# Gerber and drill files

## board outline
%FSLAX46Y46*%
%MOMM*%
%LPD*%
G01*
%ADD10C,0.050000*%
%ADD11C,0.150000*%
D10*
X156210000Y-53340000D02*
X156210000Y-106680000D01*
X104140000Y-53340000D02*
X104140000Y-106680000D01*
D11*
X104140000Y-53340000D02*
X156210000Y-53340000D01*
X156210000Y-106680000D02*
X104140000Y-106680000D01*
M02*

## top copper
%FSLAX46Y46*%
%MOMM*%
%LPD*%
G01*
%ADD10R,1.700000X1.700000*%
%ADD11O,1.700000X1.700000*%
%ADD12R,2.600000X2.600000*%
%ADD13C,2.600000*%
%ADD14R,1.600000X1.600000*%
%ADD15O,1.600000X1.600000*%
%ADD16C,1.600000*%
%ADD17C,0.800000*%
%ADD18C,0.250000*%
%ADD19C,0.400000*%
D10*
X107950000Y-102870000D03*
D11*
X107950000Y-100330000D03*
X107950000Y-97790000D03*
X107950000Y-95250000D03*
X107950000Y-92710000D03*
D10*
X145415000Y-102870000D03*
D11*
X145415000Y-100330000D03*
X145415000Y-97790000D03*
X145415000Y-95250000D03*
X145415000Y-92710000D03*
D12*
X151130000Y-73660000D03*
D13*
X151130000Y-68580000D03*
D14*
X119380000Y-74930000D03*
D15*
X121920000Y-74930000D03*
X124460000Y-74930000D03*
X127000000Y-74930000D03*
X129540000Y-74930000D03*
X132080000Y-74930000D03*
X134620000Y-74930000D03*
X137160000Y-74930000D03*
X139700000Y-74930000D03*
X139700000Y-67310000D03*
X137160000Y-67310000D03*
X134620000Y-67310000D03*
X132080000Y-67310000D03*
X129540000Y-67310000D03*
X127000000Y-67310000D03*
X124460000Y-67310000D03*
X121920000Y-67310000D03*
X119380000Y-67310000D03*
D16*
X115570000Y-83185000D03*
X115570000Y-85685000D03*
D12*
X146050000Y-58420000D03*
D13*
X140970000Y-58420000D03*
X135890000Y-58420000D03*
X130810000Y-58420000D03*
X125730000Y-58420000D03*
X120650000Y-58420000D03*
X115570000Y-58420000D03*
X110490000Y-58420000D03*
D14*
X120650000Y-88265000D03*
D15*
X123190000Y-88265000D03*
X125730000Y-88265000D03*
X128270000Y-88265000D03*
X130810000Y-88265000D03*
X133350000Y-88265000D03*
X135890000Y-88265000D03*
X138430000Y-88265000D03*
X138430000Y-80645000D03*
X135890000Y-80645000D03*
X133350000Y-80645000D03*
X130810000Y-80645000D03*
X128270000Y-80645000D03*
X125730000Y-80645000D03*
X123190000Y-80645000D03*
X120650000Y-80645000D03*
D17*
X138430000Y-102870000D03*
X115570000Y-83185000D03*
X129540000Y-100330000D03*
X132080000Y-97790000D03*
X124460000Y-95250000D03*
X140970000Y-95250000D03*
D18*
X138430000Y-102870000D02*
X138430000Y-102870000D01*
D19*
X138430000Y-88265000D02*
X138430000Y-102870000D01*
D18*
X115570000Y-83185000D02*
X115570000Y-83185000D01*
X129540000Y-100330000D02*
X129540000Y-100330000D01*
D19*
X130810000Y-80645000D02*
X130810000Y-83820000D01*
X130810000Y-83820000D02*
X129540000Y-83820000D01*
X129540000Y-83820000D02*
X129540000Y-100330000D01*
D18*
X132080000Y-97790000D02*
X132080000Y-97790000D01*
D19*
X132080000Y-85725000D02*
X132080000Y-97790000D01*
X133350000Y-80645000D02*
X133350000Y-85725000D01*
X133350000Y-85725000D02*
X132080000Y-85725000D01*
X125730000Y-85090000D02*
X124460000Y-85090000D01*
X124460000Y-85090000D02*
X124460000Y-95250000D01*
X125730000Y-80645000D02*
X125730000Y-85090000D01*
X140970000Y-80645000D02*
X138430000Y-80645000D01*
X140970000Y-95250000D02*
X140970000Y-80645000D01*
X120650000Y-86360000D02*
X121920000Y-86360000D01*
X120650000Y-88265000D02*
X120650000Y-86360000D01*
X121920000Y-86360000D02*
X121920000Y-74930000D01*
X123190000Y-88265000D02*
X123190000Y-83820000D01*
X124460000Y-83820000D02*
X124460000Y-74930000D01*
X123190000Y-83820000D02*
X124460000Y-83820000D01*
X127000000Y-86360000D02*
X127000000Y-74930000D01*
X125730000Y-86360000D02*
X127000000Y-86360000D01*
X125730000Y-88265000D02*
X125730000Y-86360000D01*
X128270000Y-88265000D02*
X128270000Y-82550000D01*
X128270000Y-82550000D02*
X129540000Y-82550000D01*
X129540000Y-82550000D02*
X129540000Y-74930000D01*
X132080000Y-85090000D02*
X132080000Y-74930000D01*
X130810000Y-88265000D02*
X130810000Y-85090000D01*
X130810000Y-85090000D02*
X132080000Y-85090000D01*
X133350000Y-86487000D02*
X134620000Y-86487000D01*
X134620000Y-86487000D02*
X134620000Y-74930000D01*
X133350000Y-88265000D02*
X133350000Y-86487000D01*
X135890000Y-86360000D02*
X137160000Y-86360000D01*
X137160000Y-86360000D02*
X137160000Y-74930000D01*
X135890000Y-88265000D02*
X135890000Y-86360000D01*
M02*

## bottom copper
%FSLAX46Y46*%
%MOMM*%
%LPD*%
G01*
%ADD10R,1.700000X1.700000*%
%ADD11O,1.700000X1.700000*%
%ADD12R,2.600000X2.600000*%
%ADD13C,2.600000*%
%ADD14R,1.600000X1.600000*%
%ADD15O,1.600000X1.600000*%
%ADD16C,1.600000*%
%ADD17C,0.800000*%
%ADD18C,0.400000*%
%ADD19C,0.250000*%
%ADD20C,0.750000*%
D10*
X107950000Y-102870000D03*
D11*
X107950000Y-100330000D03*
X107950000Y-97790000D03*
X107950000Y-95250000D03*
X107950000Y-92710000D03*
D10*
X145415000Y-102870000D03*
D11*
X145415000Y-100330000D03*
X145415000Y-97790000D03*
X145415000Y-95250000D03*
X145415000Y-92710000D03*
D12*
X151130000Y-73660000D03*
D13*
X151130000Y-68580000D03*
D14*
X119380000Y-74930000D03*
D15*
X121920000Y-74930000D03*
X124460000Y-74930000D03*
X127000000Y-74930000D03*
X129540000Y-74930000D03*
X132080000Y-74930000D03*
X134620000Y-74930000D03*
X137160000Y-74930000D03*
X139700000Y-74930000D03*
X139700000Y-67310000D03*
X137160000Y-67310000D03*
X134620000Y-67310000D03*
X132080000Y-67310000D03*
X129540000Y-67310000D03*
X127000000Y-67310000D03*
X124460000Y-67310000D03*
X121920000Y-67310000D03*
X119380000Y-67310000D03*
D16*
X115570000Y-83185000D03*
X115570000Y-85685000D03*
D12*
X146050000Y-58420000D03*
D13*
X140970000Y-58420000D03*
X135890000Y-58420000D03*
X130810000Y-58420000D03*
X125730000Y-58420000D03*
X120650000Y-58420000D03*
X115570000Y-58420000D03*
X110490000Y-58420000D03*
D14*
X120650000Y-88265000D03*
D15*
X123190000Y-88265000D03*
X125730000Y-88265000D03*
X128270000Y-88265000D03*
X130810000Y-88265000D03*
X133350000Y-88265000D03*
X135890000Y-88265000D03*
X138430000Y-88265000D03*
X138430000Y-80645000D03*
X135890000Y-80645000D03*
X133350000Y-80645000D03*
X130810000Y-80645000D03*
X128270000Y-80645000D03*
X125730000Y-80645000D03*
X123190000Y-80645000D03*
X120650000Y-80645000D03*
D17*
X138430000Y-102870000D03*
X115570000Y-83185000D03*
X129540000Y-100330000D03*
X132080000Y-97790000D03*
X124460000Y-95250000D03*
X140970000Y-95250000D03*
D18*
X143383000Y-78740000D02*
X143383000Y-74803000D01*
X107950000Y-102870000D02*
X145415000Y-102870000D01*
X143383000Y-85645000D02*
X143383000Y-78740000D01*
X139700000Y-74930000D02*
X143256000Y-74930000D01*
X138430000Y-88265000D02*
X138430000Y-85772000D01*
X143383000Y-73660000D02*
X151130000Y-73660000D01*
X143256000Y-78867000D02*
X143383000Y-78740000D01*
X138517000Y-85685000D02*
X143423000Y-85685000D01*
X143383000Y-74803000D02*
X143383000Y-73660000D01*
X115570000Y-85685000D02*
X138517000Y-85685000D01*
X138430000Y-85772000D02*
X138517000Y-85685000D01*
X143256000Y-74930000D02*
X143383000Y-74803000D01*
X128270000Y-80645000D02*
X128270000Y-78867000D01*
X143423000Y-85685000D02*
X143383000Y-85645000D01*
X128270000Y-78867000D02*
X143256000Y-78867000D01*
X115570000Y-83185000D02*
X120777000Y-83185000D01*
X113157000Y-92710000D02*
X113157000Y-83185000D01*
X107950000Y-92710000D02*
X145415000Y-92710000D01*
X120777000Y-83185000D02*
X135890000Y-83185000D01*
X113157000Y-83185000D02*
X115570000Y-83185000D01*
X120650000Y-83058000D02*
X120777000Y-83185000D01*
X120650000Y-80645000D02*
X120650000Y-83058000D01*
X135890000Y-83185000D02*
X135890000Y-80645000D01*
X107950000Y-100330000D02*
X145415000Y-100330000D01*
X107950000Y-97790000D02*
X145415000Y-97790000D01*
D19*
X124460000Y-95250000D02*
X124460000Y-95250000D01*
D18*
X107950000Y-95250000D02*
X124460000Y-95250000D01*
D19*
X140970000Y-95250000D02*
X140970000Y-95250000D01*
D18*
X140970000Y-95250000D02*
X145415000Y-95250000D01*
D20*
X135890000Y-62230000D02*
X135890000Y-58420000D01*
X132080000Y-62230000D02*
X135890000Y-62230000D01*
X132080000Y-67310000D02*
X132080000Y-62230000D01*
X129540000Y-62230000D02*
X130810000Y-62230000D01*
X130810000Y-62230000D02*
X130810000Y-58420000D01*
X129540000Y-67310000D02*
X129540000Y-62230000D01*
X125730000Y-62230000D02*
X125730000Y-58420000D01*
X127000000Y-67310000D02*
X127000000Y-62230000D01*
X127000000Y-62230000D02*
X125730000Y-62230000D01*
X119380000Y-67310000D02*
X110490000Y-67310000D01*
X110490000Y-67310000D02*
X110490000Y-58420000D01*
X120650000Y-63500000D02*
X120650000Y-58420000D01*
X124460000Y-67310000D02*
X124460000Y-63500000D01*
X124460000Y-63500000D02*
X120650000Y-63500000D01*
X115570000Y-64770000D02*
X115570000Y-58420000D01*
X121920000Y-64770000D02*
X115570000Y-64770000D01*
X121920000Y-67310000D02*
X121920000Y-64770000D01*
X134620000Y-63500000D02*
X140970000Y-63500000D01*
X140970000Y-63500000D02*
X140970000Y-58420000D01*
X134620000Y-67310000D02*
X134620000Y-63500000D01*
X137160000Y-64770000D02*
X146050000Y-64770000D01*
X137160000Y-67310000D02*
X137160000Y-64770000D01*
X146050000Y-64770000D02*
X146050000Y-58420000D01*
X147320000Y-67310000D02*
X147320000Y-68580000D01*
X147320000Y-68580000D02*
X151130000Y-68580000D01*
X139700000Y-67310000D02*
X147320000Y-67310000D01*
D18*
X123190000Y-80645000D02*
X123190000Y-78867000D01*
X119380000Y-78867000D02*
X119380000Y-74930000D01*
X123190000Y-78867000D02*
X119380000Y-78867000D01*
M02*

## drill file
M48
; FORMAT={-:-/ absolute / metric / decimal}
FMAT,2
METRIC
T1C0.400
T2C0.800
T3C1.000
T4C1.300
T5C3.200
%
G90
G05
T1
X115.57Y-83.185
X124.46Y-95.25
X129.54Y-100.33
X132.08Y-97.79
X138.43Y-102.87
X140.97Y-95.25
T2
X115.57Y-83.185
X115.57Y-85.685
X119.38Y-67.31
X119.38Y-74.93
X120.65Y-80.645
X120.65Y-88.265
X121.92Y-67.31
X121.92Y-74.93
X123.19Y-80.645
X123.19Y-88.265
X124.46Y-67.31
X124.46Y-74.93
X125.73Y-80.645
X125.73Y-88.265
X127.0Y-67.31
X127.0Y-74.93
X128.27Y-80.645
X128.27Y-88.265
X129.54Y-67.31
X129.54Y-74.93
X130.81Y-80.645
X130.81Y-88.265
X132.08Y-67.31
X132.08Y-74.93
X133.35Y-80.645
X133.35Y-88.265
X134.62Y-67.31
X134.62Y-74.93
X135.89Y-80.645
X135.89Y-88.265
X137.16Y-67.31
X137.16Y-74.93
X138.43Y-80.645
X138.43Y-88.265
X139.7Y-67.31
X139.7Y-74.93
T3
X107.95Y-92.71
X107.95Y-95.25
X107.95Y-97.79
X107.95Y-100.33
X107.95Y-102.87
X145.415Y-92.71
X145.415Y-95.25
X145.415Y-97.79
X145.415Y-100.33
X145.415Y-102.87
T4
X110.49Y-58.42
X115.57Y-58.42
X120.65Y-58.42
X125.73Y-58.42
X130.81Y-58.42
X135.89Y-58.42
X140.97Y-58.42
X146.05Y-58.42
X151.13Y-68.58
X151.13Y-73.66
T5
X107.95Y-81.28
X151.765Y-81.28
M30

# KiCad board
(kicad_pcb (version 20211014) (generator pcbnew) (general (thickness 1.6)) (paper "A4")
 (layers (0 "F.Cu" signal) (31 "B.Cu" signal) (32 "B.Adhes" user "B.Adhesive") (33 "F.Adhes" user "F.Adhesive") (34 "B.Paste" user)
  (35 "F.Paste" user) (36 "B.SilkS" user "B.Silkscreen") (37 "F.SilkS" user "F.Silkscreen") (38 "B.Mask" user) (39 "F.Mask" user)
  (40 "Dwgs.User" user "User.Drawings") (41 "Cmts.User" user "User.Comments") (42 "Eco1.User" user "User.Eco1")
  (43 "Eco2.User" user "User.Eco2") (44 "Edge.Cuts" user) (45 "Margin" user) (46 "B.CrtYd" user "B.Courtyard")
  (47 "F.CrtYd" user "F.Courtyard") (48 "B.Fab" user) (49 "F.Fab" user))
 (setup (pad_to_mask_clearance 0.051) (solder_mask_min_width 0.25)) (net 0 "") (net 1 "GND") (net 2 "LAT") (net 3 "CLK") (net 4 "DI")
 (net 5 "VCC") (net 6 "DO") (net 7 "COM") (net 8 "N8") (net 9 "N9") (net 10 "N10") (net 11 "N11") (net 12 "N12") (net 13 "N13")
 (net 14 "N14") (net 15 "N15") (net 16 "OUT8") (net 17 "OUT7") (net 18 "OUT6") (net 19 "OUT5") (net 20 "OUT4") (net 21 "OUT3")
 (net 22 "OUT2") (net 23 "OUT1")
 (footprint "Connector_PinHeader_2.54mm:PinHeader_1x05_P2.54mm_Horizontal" (layer "F.Cu") (at 107.95 102.87 180)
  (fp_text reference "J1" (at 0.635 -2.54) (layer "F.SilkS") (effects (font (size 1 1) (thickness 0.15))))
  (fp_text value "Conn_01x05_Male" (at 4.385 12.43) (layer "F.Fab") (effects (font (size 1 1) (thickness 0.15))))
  (pad "1" thru_hole rect locked (at 0 0 180) (size 1.7 1.7) (drill 1) (layers *.Cu *.Mask) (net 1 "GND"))
  (pad "2" thru_hole oval locked (at 0 2.54 180) (size 1.7 1.7) (drill 1) (layers *.Cu *.Mask) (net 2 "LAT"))
  (pad "3" thru_hole oval locked (at 0 5.08 180) (size 1.7 1.7) (drill 1) (layers *.Cu *.Mask) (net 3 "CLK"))
  (pad "4" thru_hole oval locked (at 0 7.62 180) (size 1.7 1.7) (drill 1) (layers *.Cu *.Mask) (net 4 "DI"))
  (pad "5" thru_hole oval locked (at 0 10.16 180) (size 1.7 1.7) (drill 1) (layers *.Cu *.Mask) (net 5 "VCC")))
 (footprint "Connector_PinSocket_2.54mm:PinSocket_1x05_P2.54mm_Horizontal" (layer "F.Cu") (at 145.415 102.87 180)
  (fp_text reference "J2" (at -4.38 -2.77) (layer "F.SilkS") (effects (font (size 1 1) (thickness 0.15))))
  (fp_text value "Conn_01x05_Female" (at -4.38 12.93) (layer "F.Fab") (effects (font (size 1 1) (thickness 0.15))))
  (pad "1" thru_hole rect locked (at 0 0 180) (size 1.7 1.7) (drill 1) (layers *.Cu *.Mask) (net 1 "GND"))
  (pad "2" thru_hole oval locked (at 0 2.54 180) (size 1.7 1.7) (drill 1) (layers *.Cu *.Mask) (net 2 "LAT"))
  (pad "3" thru_hole oval locked (at 0 5.08 180) (size 1.7 1.7) (drill 1) (layers *.Cu *.Mask) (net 3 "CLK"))
  (pad "4" thru_hole oval locked (at 0 7.62 180) (size 1.7 1.7) (drill 1) (layers *.Cu *.Mask) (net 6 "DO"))
  (pad "5" thru_hole oval locked (at 0 10.16 180) (size 1.7 1.7) (drill 1) (layers *.Cu *.Mask) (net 5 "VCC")))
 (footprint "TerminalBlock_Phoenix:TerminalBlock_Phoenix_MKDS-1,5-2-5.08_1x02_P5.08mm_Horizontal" (layer "F.Cu") (at 151.13 73.66 90)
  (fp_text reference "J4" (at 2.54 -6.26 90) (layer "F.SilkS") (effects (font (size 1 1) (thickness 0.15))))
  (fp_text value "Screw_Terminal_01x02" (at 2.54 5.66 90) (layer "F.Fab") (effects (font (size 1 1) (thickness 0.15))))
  (pad "1" thru_hole rect locked (at 0 0 90) (size 2.6 2.6) (drill 1.3) (layers *.Cu *.Mask) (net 1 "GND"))
  (pad "2" thru_hole circle locked (at 5.08 0 90) (size 2.6 2.6) (drill 1.3) (layers *.Cu *.Mask) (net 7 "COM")))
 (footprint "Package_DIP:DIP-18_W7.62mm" (layer "F.Cu") (at 119.38 74.93 90)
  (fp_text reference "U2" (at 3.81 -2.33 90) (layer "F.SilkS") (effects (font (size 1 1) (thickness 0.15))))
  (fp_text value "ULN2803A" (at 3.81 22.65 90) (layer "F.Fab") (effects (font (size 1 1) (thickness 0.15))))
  (pad "1" thru_hole rect locked (at 0 0 90) (size 1.6 1.6) (drill 0.8) (layers *.Cu *.Mask) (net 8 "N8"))
  (pad "2" thru_hole oval locked (at 0 2.54 90) (size 1.6 1.6) (drill 0.8) (layers *.Cu *.Mask) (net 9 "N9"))
  (pad "3" thru_hole oval locked (at 0 5.08 90) (size 1.6 1.6) (drill 0.8) (layers *.Cu *.Mask) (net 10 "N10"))
  (pad "4" thru_hole oval locked (at 0 7.62 90) (size 1.6 1.6) (drill 0.8) (layers *.Cu *.Mask) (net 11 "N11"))
  (pad "5" thru_hole oval locked (at 0 10.16 90) (size 1.6 1.6) (drill 0.8) (layers *.Cu *.Mask) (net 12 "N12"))
  (pad "6" thru_hole oval locked (at 0 12.7 90) (size 1.6 1.6) (drill 0.8) (layers *.Cu *.Mask) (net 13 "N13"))
  (pad "7" thru_hole oval locked (at 0 15.24 90) (size 1.6 1.6) (drill 0.8) (layers *.Cu *.Mask) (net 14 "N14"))
  (pad "8" thru_hole oval locked (at 0 17.78 90) (size 1.6 1.6) (drill 0.8) (layers *.Cu *.Mask) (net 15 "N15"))
  (pad "9" thru_hole oval locked (at 0 20.32 90) (size 1.6 1.6) (drill 0.8) (layers *.Cu *.Mask) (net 1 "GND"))
  (pad "10" thru_hole oval locked (at 7.62 20.32 90) (size 1.6 1.6) (drill 0.8) (layers *.Cu *.Mask) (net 7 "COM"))
  (pad "11" thru_hole oval locked (at 7.62 17.78 90) (size 1.6 1.6) (drill 0.8) (layers *.Cu *.Mask) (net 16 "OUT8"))
  (pad "12" thru_hole oval locked (at 7.62 15.24 90) (size 1.6 1.6) (drill 0.8) (layers *.Cu *.Mask) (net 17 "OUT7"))
  (pad "13" thru_hole oval locked (at 7.62 12.7 90) (size 1.6 1.6) (drill 0.8) (layers *.Cu *.Mask) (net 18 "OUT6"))
  (pad "14" thru_hole oval locked (at 7.62 10.16 90) (size 1.6 1.6) (drill 0.8) (layers *.Cu *.Mask) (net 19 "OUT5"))
  (pad "15" thru_hole oval locked (at 7.62 7.62 90) (size 1.6 1.6) (drill 0.8) (layers *.Cu *.Mask) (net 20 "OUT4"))
  (pad "16" thru_hole oval locked (at 7.62 5.08 90) (size 1.6 1.6) (drill 0.8) (layers *.Cu *.Mask) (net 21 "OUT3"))
  (pad "17" thru_hole oval locked (at 7.62 2.54 90) (size 1.6 1.6) (drill 0.8) (layers *.Cu *.Mask) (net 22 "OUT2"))
  (pad "18" thru_hole oval locked (at 7.62 0 90) (size 1.6 1.6) (drill 0.8) (layers *.Cu *.Mask) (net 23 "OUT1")))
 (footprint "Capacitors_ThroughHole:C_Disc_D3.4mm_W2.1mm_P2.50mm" (layer "F.Cu") (at 115.57 83.185 -90)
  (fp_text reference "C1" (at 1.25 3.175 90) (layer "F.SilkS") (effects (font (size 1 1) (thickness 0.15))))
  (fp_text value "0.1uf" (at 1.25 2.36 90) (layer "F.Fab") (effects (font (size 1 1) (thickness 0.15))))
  (pad "1" thru_hole circle locked (at 0 0 270) (size 1.6 1.6) (drill 0.8) (layers *.Cu *.Mask) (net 5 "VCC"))
  (pad "2" thru_hole circle locked (at 2.5 0 270) (size 1.6 1.6) (drill 0.8) (layers *.Cu *.Mask) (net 1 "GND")))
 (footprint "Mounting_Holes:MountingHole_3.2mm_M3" (layer "F.Cu") (at 107.95 81.28)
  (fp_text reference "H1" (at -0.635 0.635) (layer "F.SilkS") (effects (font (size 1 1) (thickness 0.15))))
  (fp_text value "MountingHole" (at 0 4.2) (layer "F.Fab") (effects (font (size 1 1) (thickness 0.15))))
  (pad "" np_thru_hole circle locked (at 0 0) (size 3.2 3.2) (drill 3.2) (layers *.Cu *.Mask)))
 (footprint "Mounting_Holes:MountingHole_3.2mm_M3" (layer "F.Cu") (at 151.765 81.28)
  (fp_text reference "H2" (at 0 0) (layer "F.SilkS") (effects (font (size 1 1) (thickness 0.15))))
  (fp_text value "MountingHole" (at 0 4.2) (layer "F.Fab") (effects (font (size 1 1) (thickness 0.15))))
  (pad "" np_thru_hole circle locked (at 0 0) (size 3.2 3.2) (drill 3.2) (layers *.Cu *.Mask)))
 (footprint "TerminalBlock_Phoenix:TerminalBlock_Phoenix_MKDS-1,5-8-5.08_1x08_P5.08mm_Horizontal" (layer "F.Cu") (at 146.05 58.42 180)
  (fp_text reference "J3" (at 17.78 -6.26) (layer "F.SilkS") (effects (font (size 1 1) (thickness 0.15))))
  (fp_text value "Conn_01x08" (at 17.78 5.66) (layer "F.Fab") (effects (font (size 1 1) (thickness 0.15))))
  (pad "1" thru_hole rect locked (at 0 0 180) (size 2.6 2.6) (drill 1.3) (layers *.Cu *.Mask) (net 16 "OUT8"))
  (pad "2" thru_hole circle locked (at 5.08 0 180) (size 2.6 2.6) (drill 1.3) (layers *.Cu *.Mask) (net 17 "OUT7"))
  (pad "3" thru_hole circle locked (at 10.16 0 180) (size 2.6 2.6) (drill 1.3) (layers *.Cu *.Mask) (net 18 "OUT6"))
  (pad "4" thru_hole circle locked (at 15.24 0 180) (size 2.6 2.6) (drill 1.3) (layers *.Cu *.Mask) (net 19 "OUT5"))
  (pad "5" thru_hole circle locked (at 20.32 0 180) (size 2.6 2.6) (drill 1.3) (layers *.Cu *.Mask) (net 20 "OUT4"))
  (pad "6" thru_hole circle locked (at 25.4 0 180) (size 2.6 2.6) (drill 1.3) (layers *.Cu *.Mask) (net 21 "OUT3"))
  (pad "7" thru_hole circle locked (at 30.48 0 180) (size 2.6 2.6) (drill 1.3) (layers *.Cu *.Mask) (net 22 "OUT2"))
  (pad "8" thru_hole circle locked (at 35.56 0 180) (size 2.6 2.6) (drill 1.3) (layers *.Cu *.Mask) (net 23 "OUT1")))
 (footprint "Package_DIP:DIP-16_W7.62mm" (layer "F.Cu") (at 120.65 88.265 90)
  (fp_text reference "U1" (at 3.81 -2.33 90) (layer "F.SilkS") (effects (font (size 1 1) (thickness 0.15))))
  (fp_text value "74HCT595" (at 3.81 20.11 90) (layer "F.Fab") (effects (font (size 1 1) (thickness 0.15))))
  (pad "1" thru_hole rect locked (at 0 0 90) (size 1.6 1.6) (drill 0.8) (layers *.Cu *.Mask) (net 9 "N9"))
  (pad "2" thru_hole oval locked (at 0 2.54 90) (size 1.6 1.6) (drill 0.8) (layers *.Cu *.Mask) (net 10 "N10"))
  (pad "3" thru_hole oval locked (at 0 5.08 90) (size 1.6 1.6) (drill 0.8) (layers *.Cu *.Mask) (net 11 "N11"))
  (pad "4" thru_hole oval locked (at 0 7.62 90) (size 1.6 1.6) (drill 0.8) (layers *.Cu *.Mask) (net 12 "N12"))
  (pad "5" thru_hole oval locked (at 0 10.16 90) (size 1.6 1.6) (drill 0.8) (layers *.Cu *.Mask) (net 13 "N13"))
  (pad "6" thru_hole oval locked (at 0 12.7 90) (size 1.6 1.6) (drill 0.8) (layers *.Cu *.Mask) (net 14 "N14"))
  (pad "7" thru_hole oval locked (at 0 15.24 90) (size 1.6 1.6) (drill 0.8) (layers *.Cu *.Mask) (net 15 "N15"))
  (pad "8" thru_hole oval locked (at 0 17.78 90) (size 1.6 1.6) (drill 0.8) (layers *.Cu *.Mask) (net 1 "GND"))
  (pad "9" thru_hole oval locked (at 7.62 17.78 90) (size 1.6 1.6) (drill 0.8) (layers *.Cu *.Mask) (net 6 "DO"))
  (pad "10" thru_hole oval locked (at 7.62 15.24 90) (size 1.6 1.6) (drill 0.8) (layers *.Cu *.Mask) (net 5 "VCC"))
  (pad "11" thru_hole oval locked (at 7.62 12.7 90) (size 1.6 1.6) (drill 0.8) (layers *.Cu *.Mask) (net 3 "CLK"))
  (pad "12" thru_hole oval locked (at 7.62 10.16 90) (size 1.6 1.6) (drill 0.8) (layers *.Cu *.Mask) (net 2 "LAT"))
  (pad "13" thru_hole oval locked (at 7.62 7.62 90) (size 1.6 1.6) (drill 0.8) (layers *.Cu *.Mask) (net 1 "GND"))
  (pad "14" thru_hole oval locked (at 7.62 5.08 90) (size 1.6 1.6) (drill 0.8) (layers *.Cu *.Mask) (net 4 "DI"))
  (pad "15" thru_hole oval locked (at 7.62 2.54 90) (size 1.6 1.6) (drill 0.8) (layers *.Cu *.Mask) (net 8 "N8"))
  (pad "16" thru_hole oval locked (at 7.62 0 90) (size 1.6 1.6) (drill 0.8) (layers *.Cu *.Mask) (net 5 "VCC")))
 (gr_line (start 156.21 53.34) (end 156.21 106.68) (layer "Edge.Cuts") (width 0.05))
 (gr_line (start 104.14 53.34) (end 104.14 106.68) (layer "Edge.Cuts") (width 0.05))
 (gr_line (start 104.14 53.34) (end 156.21 53.34) (layer "Edge.Cuts") (width 0.15))
 (gr_line (start 156.21 106.68) (end 104.14 106.68) (layer "Edge.Cuts") (width 0.15))
 (segment (start 138.43 102.87) (end 138.43 102.87) (width 0.25) (layer "F.Cu") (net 1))
 (segment (start 138.43 88.265) (end 138.43 102.87) (width 0.4) (layer "F.Cu") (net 1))
 (via (at 138.43 102.87) (size 0.8) (drill 0.4) (layers "F.Cu" "B.Cu") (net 1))
 (segment (start 143.383 78.74) (end 143.383 74.803) (width 0.4) (layer "B.Cu") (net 1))
 (segment (start 107.95 102.87) (end 145.415 102.87) (width 0.4) (layer "B.Cu") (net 1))
 (segment (start 143.383 85.645) (end 143.383 78.74) (width 0.4) (layer "B.Cu") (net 1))
 (segment (start 139.7 74.93) (end 143.256 74.93) (width 0.4) (layer "B.Cu") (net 1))
 (segment (start 138.43 88.265) (end 138.43 85.772) (width 0.4) (layer "B.Cu") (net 1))
 (segment (start 143.383 73.66) (end 151.13 73.66) (width 0.4) (layer "B.Cu") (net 1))
 (segment (start 143.256 78.867) (end 143.383 78.74) (width 0.4) (layer "B.Cu") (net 1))
 (segment (start 138.517 85.685) (end 143.423 85.685) (width 0.4) (layer "B.Cu") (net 1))
 (segment (start 143.383 74.803) (end 143.383 73.66) (width 0.4) (layer "B.Cu") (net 1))
 (segment (start 115.57 85.685) (end 138.517 85.685) (width 0.4) (layer "B.Cu") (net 1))
 (segment (start 138.43 85.772) (end 138.517 85.685) (width 0.4) (layer "B.Cu") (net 1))
 (segment (start 143.256 74.93) (end 143.383 74.803) (width 0.4) (layer "B.Cu") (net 1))
 (segment (start 128.27 80.645) (end 128.27 78.867) (width 0.4) (layer "B.Cu") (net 1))
 (segment (start 143.423 85.685) (end 143.383 85.645) (width 0.4) (layer "B.Cu") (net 1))
 (segment (start 128.27 78.867) (end 143.256 78.867) (width 0.4) (layer "B.Cu") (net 1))
 (segment (start 115.57 83.185) (end 115.57 83.185) (width 0.25) (layer "F.Cu") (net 5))
 (via (at 115.57 83.185) (size 0.8) (drill 0.4) (layers "F.Cu" "B.Cu") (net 5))
 (segment (start 115.57 83.185) (end 120.777 83.185) (width 0.4) (layer "B.Cu") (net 5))
 (segment (start 113.157 92.71) (end 113.157 83.185) (width 0.4) (layer "B.Cu") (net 5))
 (segment (start 107.95 92.71) (end 145.415 92.71) (width 0.4) (layer "B.Cu") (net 5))
 (segment (start 120.777 83.185) (end 135.89 83.185) (width 0.4) (layer "B.Cu") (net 5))
 (segment (start 113.157 83.185) (end 115.57 83.185) (width 0.4) (layer "B.Cu") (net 5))
 (segment (start 120.65 83.058) (end 120.777 83.185) (width 0.4) (layer "B.Cu") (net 5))
 (segment (start 120.65 80.645) (end 120.65 83.058) (width 0.4) (layer "B.Cu") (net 5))
 (segment (start 135.89 83.185) (end 135.89 80.645) (width 0.4) (layer "B.Cu") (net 5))
 (segment (start 129.54 100.33) (end 129.54 100.33) (width 0.25) (layer "F.Cu") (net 2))
 (segment (start 130.81 80.645) (end 130.81 83.82) (width 0.4) (layer "F.Cu") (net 2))
 (segment (start 130.81 83.82) (end 129.54 83.82) (width 0.4) (layer "F.Cu") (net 2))
 (segment (start 129.54 83.82) (end 129.54 100.33) (width 0.4) (layer "F.Cu") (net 2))
 (via (at 129.54 100.33) (size 0.8) (drill 0.4) (layers "F.Cu" "B.Cu") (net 2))
 (segment (start 107.95 100.33) (end 145.415 100.33) (width 0.4) (layer "B.Cu") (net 2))
 (segment (start 132.08 97.79) (end 132.08 97.79) (width 0.25) (layer "F.Cu") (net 3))
 (segment (start 132.08 85.725) (end 132.08 97.79) (width 0.4) (layer "F.Cu") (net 3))
 (segment (start 133.35 80.645) (end 133.35 85.725) (width 0.4) (layer "F.Cu") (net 3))
 (segment (start 133.35 85.725) (end 132.08 85.725) (width 0.4) (layer "F.Cu") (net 3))
 (via (at 132.08 97.79) (size 0.8) (drill 0.4) (layers "F.Cu" "B.Cu") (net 3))
 (segment (start 107.95 97.79) (end 145.415 97.79) (width 0.4) (layer "B.Cu") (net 3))
 (segment (start 125.73 85.09) (end 124.46 85.09) (width 0.4) (layer "F.Cu") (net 4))
 (segment (start 124.46 85.09) (end 124.46 95.25) (width 0.4) (layer "F.Cu") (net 4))
 (segment (start 125.73 80.645) (end 125.73 85.09) (width 0.4) (layer "F.Cu") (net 4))
 (via (at 124.46 95.25) (size 0.8) (drill 0.4) (layers "F.Cu" "B.Cu") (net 4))
 (segment (start 124.46 95.25) (end 124.46 95.25) (width 0.25) (layer "B.Cu") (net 4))
 (segment (start 107.95 95.25) (end 124.46 95.25) (width 0.4) (layer "B.Cu") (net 4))
 (segment (start 140.97 80.645) (end 138.43 80.645) (width 0.4) (layer "F.Cu") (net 6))
 (segment (start 140.97 95.25) (end 140.97 80.645) (width 0.4) (layer "F.Cu") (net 6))
 (via (at 140.97 95.25) (size 0.8) (drill 0.4) (layers "F.Cu" "B.Cu") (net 6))
 (segment (start 140.97 95.25) (end 140.97 95.25) (width 0.25) (layer "B.Cu") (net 6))
 (segment (start 140.97 95.25) (end 145.415 95.25) (width 0.4) (layer "B.Cu") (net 6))
 (segment (start 135.89 62.23) (end 135.89 58.42) (width 0.75) (layer "B.Cu") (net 18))
 (segment (start 132.08 62.23) (end 135.89 62.23) (width 0.75) (layer "B.Cu") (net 18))
 (segment (start 132.08 67.31) (end 132.08 62.23) (width 0.75) (layer "B.Cu") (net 18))
 (segment (start 129.54 62.23) (end 130.81 62.23) (width 0.75) (layer "B.Cu") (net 19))
 (segment (start 130.81 62.23) (end 130.81 58.42) (width 0.75) (layer "B.Cu") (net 19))
 (segment (start 129.54 67.31) (end 129.54 62.23) (width 0.75) (layer "B.Cu") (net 19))
 (segment (start 125.73 62.23) (end 125.73 58.42) (width 0.75) (layer "B.Cu") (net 20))
 (segment (start 127 67.31) (end 127 62.23) (width 0.75) (layer "B.Cu") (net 20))
 (segment (start 127 62.23) (end 125.73 62.23) (width 0.75) (layer "B.Cu") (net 20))
 (segment (start 119.38 67.31) (end 110.49 67.31) (width 0.75) (layer "B.Cu") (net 23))
 (segment (start 110.49 67.31) (end 110.49 58.42) (width 0.75) (layer "B.Cu") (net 23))
 (segment (start 120.65 63.5) (end 120.65 58.42) (width 0.75) (layer "B.Cu") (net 21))
 (segment (start 124.46 67.31) (end 124.46 63.5) (width 0.75) (layer "B.Cu") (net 21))
 (segment (start 124.46 63.5) (end 120.65 63.5) (width 0.75) (layer "B.Cu") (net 21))
 (segment (start 115.57 64.77) (end 115.57 58.42) (width 0.75) (layer "B.Cu") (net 22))
 (segment (start 121.92 64.77) (end 115.57 64.77) (width 0.75) (layer "B.Cu") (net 22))
 (segment (start 121.92 67.31) (end 121.92 64.77) (width 0.75) (layer "B.Cu") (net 22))
 (segment (start 134.62 63.5) (end 140.97 63.5) (width 0.75) (layer "B.Cu") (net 17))
 (segment (start 140.97 63.5) (end 140.97 58.42) (width 0.75) (layer "B.Cu") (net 17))
 (segment (start 134.62 67.31) (end 134.62 63.5) (width 0.75) (layer "B.Cu") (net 17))
 (segment (start 137.16 64.77) (end 146.05 64.77) (width 0.75) (layer "B.Cu") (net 16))
 (segment (start 137.16 67.31) (end 137.16 64.77) (width 0.75) (layer "B.Cu") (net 16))
 (segment (start 146.05 64.77) (end 146.05 58.42) (width 0.75) (layer "B.Cu") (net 16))
 (segment (start 147.32 67.31) (end 147.32 68.58) (width 0.75) (layer "B.Cu") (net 7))
 (segment (start 147.32 68.58) (end 151.13 68.58) (width 0.75) (layer "B.Cu") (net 7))
 (segment (start 139.7 67.31) (end 147.32 67.31) (width 0.75) (layer "B.Cu") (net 7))
 (segment (start 120.65 86.36) (end 121.92 86.36) (width 0.4) (layer "F.Cu") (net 9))
 (segment (start 120.65 88.265) (end 120.65 86.36) (width 0.4) (layer "F.Cu") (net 9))
 (segment (start 121.92 86.36) (end 121.92 74.93) (width 0.4) (layer "F.Cu") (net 9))
 (segment (start 123.19 88.265) (end 123.19 83.82) (width 0.4) (layer "F.Cu") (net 10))
 (segment (start 124.46 83.82) (end 124.46 74.93) (width 0.4) (layer "F.Cu") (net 10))
 (segment (start 123.19 83.82) (end 124.46 83.82) (width 0.4) (layer "F.Cu") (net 10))
 (segment (start 127 86.36) (end 127 74.93) (width 0.4) (layer "F.Cu") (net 11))
 (segment (start 125.73 86.36) (end 127 86.36) (width 0.4) (layer "F.Cu") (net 11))
 (segment (start 125.73 88.265) (end 125.73 86.36) (width 0.4) (layer "F.Cu") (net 11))
 (segment (start 128.27 88.265) (end 128.27 82.55) (width 0.4) (layer "F.Cu") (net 12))
 (segment (start 128.27 82.55) (end 129.54 82.55) (width 0.4) (layer "F.Cu") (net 12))
 (segment (start 129.54 82.55) (end 129.54 74.93) (width 0.4) (layer "F.Cu") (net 12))
 (segment (start 132.08 85.09) (end 132.08 74.93) (width 0.4) (layer "F.Cu") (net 13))
 (segment (start 130.81 88.265) (end 130.81 85.09) (width 0.4) (layer "F.Cu") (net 13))
 (segment (start 130.81 85.09) (end 132.08 85.09) (width 0.4) (layer "F.Cu") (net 13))
 (segment (start 133.35 86.487) (end 134.62 86.487) (width 0.4) (layer "F.Cu") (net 14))
 (segment (start 134.62 86.487) (end 134.62 74.93) (width 0.4) (layer "F.Cu") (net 14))
 (segment (start 133.35 88.265) (end 133.35 86.487) (width 0.4) (layer "F.Cu") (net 14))
 (segment (start 135.89 86.36) (end 137.16 86.36) (width 0.4) (layer "F.Cu") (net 15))
 (segment (start 137.16 86.36) (end 137.16 74.93) (width 0.4) (layer "F.Cu") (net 15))
 (segment (start 135.89 88.265) (end 135.89 86.36) (width 0.4) (layer "F.Cu") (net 15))
 (segment (start 123.19 80.645) (end 123.19 78.867) (width 0.4) (layer "B.Cu") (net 8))
 (segment (start 119.38 78.867) (end 119.38 74.93) (width 0.4) (layer "B.Cu") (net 8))
 (segment (start 123.19 78.867) (end 119.38 78.867) (width 0.4) (layer "B.Cu") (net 8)))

